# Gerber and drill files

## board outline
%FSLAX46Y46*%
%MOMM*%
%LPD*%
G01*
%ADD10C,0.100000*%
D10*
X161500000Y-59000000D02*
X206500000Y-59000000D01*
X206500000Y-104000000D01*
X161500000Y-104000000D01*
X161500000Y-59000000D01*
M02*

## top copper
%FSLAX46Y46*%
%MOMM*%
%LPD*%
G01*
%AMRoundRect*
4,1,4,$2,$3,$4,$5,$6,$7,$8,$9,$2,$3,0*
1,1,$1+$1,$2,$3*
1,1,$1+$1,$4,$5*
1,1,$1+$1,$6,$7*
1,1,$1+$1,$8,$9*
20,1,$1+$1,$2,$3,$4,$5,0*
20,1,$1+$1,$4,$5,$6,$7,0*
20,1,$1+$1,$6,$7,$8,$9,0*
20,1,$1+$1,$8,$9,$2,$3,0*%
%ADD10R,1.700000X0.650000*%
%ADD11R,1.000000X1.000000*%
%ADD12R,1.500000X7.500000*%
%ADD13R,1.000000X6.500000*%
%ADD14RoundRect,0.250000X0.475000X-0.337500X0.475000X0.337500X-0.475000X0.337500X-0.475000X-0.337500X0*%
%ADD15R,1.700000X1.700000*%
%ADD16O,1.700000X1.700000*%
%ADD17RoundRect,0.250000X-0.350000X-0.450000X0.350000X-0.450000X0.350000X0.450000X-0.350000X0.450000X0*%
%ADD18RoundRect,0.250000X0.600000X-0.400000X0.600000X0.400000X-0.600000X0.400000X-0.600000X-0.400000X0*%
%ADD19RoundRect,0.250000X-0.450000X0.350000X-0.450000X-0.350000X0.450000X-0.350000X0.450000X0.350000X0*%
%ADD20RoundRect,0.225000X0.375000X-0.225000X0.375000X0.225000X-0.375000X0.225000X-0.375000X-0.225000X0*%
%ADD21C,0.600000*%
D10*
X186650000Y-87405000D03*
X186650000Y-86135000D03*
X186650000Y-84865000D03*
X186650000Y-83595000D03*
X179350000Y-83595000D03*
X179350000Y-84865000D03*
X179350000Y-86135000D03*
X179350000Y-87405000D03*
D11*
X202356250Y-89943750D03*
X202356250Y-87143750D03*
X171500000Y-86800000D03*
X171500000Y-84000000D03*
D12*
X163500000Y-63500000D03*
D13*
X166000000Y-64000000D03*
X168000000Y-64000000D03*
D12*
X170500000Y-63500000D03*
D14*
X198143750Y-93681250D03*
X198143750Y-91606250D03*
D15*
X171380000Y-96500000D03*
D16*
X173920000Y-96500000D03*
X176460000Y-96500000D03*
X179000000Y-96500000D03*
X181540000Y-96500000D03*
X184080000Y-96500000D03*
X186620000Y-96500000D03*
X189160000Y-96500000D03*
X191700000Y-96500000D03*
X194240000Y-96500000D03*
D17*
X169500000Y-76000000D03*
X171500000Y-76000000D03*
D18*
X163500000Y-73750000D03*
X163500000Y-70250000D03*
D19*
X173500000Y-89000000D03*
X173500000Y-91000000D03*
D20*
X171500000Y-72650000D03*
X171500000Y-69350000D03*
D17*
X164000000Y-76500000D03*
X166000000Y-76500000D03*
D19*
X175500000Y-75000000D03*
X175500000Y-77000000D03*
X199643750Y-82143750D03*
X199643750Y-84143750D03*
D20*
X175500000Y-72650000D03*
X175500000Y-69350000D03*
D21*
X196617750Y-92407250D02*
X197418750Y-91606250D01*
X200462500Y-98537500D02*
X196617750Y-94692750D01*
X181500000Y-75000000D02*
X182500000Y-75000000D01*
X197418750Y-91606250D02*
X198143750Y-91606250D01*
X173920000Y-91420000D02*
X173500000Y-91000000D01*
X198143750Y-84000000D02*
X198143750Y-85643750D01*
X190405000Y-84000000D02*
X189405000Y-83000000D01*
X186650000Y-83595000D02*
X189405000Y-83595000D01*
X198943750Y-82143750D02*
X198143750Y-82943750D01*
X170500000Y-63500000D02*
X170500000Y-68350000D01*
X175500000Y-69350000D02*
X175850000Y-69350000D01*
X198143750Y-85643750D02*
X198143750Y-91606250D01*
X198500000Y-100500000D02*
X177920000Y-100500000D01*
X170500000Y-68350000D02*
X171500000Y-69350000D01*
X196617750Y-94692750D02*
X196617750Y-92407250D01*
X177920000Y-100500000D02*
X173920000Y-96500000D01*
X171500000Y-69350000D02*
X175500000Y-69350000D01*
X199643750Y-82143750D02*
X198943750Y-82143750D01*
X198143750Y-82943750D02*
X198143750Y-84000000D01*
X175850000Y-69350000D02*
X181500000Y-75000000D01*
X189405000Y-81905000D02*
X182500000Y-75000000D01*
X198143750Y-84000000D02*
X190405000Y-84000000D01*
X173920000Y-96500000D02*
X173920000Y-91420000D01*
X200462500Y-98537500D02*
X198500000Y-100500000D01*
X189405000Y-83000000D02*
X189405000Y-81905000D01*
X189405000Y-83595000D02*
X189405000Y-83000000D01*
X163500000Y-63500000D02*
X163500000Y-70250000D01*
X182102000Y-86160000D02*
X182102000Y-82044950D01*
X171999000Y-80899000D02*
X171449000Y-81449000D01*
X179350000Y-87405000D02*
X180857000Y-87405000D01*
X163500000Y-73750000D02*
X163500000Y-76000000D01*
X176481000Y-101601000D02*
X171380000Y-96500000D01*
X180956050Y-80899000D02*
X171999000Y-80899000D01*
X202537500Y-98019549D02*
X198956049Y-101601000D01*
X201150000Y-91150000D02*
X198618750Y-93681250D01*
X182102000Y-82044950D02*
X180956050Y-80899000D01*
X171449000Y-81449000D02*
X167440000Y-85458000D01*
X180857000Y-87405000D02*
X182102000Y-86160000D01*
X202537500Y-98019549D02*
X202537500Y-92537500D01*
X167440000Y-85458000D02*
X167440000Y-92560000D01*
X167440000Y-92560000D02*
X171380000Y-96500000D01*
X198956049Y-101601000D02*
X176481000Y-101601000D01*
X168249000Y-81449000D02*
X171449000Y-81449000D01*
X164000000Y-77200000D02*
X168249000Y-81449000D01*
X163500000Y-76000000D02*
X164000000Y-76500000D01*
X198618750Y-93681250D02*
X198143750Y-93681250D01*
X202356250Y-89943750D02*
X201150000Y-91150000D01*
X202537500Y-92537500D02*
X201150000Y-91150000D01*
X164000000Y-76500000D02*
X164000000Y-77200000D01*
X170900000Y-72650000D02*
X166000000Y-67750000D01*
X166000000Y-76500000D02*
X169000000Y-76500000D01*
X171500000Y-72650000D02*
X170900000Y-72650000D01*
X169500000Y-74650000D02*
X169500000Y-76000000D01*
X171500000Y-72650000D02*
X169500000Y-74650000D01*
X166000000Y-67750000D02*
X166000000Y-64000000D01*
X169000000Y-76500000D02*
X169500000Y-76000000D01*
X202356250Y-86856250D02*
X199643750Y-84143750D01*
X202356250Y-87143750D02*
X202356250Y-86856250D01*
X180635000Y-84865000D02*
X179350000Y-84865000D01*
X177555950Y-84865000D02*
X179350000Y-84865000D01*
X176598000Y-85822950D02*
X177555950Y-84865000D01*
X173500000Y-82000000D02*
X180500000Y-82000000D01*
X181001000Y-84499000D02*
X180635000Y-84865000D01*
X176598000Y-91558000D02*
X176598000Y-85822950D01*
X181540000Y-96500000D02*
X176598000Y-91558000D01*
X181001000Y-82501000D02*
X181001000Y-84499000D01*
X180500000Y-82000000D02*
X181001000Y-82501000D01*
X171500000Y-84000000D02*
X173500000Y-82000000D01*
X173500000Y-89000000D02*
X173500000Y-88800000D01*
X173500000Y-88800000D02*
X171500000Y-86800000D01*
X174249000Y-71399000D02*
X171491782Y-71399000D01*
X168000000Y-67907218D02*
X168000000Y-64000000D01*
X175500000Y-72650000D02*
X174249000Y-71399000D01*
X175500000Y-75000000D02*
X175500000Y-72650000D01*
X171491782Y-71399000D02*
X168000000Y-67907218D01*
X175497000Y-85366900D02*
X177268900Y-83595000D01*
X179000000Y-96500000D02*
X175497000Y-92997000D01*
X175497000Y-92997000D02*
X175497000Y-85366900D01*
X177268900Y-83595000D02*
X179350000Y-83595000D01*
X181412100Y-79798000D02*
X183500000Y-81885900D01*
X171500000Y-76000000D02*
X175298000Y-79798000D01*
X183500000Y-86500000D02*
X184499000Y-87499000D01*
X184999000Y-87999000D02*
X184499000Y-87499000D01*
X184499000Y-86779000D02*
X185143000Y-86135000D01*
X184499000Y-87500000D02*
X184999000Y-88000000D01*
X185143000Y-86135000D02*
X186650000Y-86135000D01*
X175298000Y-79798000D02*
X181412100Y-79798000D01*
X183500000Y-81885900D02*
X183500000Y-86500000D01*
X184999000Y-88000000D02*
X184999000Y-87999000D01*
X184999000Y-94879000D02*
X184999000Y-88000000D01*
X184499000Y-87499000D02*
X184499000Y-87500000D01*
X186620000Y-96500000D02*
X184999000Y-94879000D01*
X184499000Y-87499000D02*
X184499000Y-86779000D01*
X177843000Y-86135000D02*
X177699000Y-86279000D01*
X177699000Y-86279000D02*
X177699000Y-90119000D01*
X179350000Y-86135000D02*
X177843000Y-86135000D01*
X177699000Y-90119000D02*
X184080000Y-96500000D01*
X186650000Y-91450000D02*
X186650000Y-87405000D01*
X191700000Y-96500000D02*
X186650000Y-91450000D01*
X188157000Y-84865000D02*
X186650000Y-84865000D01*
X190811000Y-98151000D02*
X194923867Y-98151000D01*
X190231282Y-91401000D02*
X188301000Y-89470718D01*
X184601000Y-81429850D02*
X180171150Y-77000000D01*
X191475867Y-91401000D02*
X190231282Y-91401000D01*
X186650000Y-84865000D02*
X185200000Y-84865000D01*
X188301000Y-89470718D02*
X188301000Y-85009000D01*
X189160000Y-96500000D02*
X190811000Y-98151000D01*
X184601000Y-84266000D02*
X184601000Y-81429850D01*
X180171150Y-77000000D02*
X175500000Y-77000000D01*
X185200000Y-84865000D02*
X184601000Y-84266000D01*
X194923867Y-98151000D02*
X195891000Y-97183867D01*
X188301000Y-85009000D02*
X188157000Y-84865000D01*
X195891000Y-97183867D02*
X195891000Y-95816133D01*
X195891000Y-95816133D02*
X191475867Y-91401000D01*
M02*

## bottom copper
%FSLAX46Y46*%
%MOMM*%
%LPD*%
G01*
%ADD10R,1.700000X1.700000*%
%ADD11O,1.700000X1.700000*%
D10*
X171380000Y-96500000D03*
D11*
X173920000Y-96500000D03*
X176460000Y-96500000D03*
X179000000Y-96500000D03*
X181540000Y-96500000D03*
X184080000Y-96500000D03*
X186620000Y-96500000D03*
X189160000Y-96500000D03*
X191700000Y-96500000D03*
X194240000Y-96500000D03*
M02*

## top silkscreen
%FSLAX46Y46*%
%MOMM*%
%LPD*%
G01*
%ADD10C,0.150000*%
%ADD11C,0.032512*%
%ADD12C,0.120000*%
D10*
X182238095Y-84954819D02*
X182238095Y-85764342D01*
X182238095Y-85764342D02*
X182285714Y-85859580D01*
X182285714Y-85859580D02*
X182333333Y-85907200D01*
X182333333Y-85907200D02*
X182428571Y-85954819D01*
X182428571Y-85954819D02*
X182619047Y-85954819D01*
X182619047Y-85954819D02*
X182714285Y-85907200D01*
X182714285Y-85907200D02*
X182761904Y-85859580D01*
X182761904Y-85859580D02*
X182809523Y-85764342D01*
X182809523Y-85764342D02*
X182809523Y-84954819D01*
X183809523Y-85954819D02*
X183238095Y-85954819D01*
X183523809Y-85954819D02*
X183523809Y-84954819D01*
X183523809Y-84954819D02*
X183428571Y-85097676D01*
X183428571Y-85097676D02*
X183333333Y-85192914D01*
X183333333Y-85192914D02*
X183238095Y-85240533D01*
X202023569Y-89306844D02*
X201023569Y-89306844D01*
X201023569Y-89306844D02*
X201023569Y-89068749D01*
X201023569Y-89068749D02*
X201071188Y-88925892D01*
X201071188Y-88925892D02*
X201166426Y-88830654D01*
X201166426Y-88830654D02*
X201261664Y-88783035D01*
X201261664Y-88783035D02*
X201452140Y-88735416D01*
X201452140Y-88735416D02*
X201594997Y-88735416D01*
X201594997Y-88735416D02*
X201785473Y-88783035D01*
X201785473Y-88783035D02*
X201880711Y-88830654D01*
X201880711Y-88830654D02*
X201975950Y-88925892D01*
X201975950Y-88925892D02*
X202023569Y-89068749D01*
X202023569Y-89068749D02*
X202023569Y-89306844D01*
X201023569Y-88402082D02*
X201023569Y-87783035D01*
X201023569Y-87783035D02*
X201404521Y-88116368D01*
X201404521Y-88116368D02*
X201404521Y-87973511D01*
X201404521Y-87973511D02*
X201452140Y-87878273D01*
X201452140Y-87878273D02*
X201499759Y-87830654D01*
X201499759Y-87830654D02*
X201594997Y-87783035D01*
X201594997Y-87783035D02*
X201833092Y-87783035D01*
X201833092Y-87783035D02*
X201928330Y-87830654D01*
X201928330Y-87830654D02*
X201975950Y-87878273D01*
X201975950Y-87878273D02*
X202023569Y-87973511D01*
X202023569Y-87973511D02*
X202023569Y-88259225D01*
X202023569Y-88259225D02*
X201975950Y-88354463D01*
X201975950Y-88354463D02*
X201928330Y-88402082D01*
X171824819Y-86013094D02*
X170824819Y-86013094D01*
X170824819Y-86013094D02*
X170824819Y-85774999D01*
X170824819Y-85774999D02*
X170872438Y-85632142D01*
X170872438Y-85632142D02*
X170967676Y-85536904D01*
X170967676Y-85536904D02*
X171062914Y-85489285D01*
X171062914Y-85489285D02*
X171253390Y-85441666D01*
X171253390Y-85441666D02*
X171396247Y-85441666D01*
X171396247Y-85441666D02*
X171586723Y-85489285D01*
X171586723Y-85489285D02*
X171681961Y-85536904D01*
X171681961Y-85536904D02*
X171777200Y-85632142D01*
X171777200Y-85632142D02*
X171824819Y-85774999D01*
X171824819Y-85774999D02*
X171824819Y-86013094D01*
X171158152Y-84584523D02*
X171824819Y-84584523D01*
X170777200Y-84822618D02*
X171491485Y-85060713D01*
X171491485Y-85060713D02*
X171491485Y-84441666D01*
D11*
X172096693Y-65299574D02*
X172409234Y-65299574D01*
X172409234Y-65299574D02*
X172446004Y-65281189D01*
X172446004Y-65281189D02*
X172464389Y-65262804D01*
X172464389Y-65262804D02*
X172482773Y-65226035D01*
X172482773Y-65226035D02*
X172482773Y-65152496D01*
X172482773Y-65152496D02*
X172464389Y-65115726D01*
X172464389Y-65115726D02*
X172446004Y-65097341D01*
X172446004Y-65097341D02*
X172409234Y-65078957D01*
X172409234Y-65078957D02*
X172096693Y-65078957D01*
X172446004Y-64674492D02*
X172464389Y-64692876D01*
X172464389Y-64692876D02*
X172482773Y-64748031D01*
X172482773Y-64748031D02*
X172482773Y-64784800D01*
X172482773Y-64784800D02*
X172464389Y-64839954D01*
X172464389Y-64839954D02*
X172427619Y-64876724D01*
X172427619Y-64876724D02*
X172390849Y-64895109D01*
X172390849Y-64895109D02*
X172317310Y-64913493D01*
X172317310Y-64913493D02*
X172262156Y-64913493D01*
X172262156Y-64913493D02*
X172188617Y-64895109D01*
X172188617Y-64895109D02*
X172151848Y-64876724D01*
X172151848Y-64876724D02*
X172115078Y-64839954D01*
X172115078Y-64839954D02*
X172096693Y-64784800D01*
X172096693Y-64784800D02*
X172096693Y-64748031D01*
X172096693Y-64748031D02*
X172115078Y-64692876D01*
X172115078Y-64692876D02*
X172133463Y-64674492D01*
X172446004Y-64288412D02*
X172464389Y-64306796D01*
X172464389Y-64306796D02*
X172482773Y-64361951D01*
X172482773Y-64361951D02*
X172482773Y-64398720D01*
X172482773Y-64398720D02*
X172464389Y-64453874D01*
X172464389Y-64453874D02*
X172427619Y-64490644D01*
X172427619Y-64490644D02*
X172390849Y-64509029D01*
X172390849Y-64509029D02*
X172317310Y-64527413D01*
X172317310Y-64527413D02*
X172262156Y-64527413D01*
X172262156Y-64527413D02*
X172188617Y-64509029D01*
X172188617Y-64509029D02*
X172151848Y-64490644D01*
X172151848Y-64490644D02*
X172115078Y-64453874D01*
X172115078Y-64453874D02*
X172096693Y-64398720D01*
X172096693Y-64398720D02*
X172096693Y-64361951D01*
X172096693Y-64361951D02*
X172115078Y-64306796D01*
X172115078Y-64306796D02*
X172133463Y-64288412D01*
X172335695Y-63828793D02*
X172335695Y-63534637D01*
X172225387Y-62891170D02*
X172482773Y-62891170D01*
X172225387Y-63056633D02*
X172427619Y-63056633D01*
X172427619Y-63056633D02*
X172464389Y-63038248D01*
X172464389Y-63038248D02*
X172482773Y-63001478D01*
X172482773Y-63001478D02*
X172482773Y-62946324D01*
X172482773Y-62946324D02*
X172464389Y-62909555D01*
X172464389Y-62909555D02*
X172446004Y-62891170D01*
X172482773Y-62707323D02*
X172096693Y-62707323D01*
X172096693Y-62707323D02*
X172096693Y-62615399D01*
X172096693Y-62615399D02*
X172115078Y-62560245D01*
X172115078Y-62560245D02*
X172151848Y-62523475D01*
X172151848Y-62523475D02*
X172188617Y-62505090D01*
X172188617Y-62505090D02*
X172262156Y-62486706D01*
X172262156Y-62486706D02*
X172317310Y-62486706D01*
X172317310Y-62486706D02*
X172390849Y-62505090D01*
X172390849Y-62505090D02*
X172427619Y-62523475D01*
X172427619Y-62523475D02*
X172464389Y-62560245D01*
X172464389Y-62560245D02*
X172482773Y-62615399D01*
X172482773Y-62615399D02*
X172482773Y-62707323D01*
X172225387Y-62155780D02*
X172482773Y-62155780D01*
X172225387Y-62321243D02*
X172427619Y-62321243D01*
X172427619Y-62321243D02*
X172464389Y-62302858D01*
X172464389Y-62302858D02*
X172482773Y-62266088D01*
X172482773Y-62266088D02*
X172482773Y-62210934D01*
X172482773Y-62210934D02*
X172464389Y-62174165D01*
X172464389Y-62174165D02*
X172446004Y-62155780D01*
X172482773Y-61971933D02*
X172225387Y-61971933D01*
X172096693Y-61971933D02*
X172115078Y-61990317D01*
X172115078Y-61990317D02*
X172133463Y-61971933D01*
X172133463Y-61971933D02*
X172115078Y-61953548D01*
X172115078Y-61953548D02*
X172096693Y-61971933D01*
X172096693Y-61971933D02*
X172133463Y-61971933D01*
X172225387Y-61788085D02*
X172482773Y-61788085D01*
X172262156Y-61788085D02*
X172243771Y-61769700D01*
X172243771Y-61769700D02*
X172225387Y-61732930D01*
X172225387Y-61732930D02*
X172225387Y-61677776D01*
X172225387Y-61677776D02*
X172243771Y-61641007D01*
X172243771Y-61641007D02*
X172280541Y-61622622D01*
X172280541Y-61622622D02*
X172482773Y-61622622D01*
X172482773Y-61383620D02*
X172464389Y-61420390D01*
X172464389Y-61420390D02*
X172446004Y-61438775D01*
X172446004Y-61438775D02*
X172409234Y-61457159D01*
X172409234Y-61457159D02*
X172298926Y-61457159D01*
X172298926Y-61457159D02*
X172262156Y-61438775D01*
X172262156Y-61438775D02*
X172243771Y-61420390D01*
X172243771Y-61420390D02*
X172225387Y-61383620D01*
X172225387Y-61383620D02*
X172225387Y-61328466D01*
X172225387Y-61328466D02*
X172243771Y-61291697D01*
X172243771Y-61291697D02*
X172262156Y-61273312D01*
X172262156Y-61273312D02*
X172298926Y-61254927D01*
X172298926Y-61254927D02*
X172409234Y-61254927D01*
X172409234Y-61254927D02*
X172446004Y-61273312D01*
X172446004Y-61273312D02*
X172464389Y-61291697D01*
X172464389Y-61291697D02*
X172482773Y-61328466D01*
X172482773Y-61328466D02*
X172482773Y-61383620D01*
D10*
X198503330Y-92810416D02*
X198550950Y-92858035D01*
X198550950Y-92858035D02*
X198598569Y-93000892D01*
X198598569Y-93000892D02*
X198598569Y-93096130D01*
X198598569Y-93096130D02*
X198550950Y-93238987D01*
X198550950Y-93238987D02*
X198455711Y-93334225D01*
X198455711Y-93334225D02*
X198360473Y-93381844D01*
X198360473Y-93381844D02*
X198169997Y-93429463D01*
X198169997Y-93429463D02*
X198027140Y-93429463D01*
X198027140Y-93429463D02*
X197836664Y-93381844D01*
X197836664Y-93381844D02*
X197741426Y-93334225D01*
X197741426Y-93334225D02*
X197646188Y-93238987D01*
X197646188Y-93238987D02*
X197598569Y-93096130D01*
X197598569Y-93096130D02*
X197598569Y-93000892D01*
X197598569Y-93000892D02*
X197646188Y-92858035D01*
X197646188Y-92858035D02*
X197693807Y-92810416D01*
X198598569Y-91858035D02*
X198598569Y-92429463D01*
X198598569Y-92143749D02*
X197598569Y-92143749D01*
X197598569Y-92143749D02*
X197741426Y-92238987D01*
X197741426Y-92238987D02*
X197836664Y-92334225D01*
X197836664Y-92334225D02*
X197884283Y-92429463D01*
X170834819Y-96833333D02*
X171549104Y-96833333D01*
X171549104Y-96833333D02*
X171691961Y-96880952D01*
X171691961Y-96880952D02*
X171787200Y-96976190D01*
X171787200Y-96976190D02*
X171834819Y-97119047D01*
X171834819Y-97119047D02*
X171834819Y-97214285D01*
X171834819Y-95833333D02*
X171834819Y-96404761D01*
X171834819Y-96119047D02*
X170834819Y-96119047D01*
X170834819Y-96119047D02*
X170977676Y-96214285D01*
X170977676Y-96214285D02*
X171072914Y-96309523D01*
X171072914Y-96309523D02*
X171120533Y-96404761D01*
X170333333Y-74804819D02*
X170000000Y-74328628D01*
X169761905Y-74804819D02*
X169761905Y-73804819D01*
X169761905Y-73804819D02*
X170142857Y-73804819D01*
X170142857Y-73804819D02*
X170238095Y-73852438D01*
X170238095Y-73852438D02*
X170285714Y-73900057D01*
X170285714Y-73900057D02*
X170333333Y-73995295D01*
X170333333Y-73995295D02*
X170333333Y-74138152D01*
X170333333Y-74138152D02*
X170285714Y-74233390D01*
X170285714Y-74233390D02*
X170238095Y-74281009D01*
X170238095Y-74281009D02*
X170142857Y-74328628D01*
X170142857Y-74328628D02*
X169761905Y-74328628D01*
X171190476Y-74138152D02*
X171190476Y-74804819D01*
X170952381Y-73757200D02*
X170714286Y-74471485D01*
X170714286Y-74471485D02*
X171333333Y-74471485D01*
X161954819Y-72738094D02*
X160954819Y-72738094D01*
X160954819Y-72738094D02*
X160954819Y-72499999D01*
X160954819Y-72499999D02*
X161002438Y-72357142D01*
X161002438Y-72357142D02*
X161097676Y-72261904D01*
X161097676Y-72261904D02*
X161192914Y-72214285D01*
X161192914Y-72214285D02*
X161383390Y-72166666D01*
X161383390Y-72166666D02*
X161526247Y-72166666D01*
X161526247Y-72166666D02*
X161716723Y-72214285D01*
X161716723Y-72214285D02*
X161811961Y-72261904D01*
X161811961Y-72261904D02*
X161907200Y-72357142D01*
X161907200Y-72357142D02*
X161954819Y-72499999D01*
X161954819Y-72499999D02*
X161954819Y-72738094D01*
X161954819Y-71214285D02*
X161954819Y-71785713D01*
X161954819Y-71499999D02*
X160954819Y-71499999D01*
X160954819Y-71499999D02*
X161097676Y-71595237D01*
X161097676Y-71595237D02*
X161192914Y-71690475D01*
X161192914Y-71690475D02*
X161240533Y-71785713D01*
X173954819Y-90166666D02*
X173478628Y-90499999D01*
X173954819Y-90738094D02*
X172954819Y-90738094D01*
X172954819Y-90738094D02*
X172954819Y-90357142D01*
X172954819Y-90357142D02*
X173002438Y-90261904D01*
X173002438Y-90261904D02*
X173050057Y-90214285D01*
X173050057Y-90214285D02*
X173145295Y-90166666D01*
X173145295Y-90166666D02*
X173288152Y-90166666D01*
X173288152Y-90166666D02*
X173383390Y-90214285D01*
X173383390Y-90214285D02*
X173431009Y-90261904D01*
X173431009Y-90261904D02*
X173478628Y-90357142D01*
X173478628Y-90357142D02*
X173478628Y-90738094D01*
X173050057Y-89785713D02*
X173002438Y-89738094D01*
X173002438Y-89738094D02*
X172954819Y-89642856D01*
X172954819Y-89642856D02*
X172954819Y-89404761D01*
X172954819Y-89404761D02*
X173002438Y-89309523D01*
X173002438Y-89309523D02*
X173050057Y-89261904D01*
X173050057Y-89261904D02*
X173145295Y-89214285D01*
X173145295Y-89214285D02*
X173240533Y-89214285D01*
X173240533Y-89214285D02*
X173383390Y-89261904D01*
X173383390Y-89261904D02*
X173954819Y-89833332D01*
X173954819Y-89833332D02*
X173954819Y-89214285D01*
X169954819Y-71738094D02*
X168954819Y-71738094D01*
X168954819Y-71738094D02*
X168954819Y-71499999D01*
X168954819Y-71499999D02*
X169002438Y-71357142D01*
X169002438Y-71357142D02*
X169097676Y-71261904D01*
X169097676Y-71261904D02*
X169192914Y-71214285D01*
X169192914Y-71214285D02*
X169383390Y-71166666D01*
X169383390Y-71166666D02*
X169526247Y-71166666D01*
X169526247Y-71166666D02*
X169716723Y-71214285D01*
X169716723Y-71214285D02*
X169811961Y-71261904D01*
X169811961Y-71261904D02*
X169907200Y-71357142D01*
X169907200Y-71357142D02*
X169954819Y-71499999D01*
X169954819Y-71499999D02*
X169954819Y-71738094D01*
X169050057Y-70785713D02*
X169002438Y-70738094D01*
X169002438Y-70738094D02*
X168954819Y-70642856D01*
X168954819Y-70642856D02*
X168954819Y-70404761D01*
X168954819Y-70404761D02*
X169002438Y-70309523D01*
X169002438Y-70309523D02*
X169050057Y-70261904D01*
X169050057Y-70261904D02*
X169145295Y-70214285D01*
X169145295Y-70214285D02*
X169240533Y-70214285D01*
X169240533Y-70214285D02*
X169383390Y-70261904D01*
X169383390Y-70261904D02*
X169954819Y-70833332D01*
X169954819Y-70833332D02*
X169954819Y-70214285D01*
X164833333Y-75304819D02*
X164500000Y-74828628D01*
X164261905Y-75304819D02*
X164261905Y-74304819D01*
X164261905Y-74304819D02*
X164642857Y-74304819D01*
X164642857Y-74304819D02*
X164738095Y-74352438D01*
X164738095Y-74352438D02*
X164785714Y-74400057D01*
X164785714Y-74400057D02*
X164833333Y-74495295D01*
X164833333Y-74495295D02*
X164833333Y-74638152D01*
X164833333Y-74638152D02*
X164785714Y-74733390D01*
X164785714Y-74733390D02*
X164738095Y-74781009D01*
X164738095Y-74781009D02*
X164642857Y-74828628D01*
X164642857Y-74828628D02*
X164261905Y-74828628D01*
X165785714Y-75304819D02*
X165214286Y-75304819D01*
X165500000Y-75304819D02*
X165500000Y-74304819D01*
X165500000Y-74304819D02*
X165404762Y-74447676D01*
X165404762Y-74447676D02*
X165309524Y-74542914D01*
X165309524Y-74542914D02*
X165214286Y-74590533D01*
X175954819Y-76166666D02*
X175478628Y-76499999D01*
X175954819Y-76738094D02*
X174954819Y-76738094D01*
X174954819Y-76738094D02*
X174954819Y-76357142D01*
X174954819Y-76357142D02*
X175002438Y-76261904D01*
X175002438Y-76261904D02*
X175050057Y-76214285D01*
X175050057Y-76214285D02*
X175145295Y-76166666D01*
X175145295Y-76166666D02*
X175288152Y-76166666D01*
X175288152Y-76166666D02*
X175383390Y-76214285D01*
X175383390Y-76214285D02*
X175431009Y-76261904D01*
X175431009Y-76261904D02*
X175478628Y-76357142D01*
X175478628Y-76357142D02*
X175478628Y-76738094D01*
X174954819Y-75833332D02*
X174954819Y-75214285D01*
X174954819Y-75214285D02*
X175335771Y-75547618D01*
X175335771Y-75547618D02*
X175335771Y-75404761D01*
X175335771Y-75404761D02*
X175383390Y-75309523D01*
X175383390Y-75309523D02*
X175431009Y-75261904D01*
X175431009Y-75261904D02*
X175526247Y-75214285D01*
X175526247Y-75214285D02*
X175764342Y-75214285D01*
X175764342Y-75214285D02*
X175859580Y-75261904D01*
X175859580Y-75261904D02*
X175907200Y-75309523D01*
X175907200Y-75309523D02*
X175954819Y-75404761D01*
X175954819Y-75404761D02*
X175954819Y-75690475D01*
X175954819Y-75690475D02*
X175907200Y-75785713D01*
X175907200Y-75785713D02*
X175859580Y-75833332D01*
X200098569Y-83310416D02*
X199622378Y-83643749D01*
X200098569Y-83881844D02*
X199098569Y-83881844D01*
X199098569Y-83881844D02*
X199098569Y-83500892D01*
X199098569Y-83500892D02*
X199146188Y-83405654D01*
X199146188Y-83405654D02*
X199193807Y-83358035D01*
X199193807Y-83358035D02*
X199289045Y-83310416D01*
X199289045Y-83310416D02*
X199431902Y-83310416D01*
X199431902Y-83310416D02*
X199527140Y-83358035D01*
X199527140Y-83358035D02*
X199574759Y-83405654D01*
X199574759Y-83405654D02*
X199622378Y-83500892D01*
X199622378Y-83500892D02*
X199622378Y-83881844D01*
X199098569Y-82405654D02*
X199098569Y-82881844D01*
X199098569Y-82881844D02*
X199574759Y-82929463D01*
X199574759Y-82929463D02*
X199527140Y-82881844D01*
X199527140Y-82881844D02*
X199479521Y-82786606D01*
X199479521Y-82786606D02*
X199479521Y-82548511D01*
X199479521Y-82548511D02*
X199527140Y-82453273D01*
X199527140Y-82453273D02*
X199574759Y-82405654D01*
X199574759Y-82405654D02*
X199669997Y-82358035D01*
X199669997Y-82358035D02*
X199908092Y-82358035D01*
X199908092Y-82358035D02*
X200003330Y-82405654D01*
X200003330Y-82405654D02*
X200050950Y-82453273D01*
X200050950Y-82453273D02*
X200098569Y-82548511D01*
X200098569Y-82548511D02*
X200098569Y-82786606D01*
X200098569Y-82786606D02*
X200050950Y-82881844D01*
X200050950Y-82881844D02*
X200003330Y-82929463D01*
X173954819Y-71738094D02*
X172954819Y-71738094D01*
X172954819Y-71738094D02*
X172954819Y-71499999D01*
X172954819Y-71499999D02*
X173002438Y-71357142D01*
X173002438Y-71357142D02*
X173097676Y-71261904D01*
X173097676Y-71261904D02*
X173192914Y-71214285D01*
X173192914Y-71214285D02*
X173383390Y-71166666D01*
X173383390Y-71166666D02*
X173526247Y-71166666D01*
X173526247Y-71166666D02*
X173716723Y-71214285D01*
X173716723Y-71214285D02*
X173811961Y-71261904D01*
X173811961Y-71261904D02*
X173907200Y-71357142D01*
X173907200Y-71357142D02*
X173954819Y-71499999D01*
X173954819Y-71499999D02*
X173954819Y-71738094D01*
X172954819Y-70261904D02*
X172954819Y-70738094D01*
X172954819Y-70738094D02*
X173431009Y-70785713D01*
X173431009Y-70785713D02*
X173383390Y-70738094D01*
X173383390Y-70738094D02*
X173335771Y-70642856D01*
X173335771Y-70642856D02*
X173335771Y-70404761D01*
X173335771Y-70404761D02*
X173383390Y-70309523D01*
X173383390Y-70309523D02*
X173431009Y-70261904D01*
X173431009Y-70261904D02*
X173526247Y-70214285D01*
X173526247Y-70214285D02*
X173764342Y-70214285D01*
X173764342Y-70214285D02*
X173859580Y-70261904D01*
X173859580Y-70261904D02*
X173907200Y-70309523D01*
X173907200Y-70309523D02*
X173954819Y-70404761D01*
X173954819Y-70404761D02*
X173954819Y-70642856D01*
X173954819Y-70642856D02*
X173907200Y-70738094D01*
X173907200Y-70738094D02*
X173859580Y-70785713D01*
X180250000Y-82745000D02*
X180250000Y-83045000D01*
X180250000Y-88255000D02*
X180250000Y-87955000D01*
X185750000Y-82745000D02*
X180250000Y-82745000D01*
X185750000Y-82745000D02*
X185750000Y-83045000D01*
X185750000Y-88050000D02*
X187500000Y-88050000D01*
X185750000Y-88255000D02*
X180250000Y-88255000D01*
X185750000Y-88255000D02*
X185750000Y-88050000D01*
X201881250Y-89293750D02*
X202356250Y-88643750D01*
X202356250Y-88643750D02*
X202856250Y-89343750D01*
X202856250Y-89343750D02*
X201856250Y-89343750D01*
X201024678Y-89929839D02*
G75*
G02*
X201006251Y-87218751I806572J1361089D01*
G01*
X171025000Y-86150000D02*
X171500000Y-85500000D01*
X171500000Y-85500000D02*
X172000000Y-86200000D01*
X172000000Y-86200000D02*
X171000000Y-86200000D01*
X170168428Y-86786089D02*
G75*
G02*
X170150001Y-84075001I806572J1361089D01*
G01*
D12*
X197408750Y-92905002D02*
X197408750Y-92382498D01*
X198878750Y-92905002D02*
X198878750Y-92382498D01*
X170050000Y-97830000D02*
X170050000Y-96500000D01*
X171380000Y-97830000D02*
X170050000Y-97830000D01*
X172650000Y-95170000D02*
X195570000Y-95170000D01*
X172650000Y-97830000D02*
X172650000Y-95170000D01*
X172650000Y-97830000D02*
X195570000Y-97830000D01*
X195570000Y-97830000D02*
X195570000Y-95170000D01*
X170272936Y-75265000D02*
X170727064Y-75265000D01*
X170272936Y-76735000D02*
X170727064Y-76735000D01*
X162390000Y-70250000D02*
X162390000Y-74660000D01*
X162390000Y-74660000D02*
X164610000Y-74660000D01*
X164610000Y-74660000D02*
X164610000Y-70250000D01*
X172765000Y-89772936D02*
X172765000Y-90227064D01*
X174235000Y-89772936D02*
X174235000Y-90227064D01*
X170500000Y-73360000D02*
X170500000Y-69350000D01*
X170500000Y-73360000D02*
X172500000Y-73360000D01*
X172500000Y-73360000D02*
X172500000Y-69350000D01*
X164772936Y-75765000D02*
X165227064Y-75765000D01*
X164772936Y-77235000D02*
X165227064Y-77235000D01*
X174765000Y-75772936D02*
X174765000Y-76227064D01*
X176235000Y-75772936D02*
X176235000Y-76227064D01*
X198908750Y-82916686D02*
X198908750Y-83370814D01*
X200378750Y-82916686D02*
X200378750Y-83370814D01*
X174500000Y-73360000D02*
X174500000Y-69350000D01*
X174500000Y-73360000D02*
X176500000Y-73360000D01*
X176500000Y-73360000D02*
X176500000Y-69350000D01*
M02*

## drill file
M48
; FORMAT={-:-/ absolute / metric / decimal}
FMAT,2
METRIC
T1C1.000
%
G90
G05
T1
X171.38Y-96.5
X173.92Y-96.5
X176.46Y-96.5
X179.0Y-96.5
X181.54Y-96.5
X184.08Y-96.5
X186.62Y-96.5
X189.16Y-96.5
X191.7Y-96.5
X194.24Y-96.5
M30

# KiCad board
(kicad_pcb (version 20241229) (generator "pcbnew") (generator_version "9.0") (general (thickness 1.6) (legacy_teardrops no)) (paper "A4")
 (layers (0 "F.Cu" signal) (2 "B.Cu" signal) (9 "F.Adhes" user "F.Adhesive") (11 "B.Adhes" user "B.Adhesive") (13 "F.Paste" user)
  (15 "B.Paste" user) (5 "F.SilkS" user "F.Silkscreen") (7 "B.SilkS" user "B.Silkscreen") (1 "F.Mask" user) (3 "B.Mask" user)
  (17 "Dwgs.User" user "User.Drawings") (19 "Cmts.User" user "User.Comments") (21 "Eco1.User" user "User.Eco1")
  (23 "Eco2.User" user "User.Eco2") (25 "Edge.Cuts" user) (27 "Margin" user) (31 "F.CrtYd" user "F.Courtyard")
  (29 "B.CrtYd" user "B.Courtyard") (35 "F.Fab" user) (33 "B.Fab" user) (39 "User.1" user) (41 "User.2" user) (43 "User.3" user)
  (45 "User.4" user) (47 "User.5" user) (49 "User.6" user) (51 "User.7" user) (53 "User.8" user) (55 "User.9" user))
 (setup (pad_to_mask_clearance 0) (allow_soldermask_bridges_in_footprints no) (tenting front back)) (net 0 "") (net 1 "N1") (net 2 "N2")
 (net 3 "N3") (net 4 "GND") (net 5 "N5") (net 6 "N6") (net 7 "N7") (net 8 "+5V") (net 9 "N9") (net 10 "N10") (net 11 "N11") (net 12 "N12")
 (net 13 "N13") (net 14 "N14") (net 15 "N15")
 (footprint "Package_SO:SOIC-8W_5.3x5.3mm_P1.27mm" (layer "F.Cu") (at 183 85.5 180)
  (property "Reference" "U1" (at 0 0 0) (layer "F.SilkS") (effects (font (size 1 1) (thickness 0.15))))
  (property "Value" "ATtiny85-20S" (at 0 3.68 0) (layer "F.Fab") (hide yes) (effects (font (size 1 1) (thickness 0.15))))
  (fp_line (start 2.75 2.755) (end 2.75 2.455) (stroke (width 0.15) (type solid)) (layer "F.SilkS"))
  (fp_line (start 2.75 -2.755) (end 2.75 -2.455) (stroke (width 0.15) (type solid)) (layer "F.SilkS"))
  (fp_line (start -2.75 2.755) (end 2.75 2.755) (stroke (width 0.15) (type solid)) (layer "F.SilkS"))
  (fp_line (start -2.75 2.755) (end -2.75 2.455) (stroke (width 0.15) (type solid)) (layer "F.SilkS"))
  (fp_line (start -2.75 -2.55) (end -4.5 -2.55) (stroke (width 0.15) (type solid)) (layer "F.SilkS"))
  (fp_line (start -2.75 -2.755) (end 2.75 -2.755) (stroke (width 0.15) (type solid)) (layer "F.SilkS"))
  (fp_line (start -2.75 -2.755) (end -2.75 -2.55) (stroke (width 0.15) (type solid)) (layer "F.SilkS"))
  (pad "1" smd rect (at -3.65 -1.905 180) (size 1.7 0.65) (layers "F.Cu" "F.Mask" "F.Paste") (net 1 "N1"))
  (pad "2" smd rect (at -3.65 -0.635 180) (size 1.7 0.65) (layers "F.Cu" "F.Mask" "F.Paste") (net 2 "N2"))
  (pad "3" smd rect (at -3.65 0.635 180) (size 1.7 0.65) (layers "F.Cu" "F.Mask" "F.Paste") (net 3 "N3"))
  (pad "4" smd rect (at -3.65 1.905 180) (size 1.7 0.65) (layers "F.Cu" "F.Mask" "F.Paste") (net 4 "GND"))
  (pad "5" smd rect (at 3.65 1.905 180) (size 1.7 0.65) (layers "F.Cu" "F.Mask" "F.Paste") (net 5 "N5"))
  (pad "6" smd rect (at 3.65 0.635 180) (size 1.7 0.65) (layers "F.Cu" "F.Mask" "F.Paste") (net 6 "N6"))
  (pad "7" smd rect (at 3.65 -0.635 180) (size 1.7 0.65) (layers "F.Cu" "F.Mask" "F.Paste") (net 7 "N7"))
  (pad "8" smd rect (at 3.65 -1.905 180) (size 1.7 0.65) (layers "F.Cu" "F.Mask" "F.Paste") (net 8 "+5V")))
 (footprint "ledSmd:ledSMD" (layer "F.Cu") (at 202.35625 88.14375 90)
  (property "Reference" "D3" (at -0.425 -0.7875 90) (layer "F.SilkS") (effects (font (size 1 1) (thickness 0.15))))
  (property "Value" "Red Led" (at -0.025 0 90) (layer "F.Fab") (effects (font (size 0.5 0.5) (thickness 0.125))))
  (fp_line (start -1.15 -0.475) (end -0.5 0) (stroke (width 0.15) (type solid)) (layer "F.SilkS"))
  (fp_line (start -0.5 0) (end -1.2 0.5) (stroke (width 0.15) (type solid)) (layer "F.SilkS"))
  (fp_line (start -1.2 0.5) (end -1.2 -0.5) (stroke (width 0.15) (type solid)) (layer "F.SilkS"))
  (fp_arc (start -1.786089 -1.331572) (mid -0.435753 -2.107089) (end 0.924999 -1.349999) (stroke (width 0.15) (type solid))
   (layer "F.SilkS"))
  (pad "1" smd rect (at -1.8 0 90) (size 1 1) (layers "F.Cu" "F.Mask" "F.Paste") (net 8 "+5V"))
  (pad "2" smd rect (at 1 0 90) (size 1 1) (layers "F.Cu" "F.Mask" "F.Paste") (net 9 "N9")))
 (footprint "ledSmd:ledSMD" (layer "F.Cu") (at 171.5 85 90)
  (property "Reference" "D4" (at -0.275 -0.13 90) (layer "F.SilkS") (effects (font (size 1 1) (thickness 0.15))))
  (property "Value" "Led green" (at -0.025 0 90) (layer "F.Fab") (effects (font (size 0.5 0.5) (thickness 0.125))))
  (fp_line (start -1.15 -0.475) (end -0.5 0) (stroke (width 0.15) (type solid)) (layer "F.SilkS"))
  (fp_line (start -0.5 0) (end -1.2 0.5) (stroke (width 0.15) (type solid)) (layer "F.SilkS"))
  (fp_line (start -1.2 0.5) (end -1.2 -0.5) (stroke (width 0.15) (type solid)) (layer "F.SilkS"))
  (fp_arc (start -1.786089 -1.331572) (mid -0.435753 -2.107089) (end 0.924999 -1.349999) (stroke (width 0.15) (type solid))
   (layer "F.SilkS"))
  (pad "1" smd rect (at -1.8 0 90) (size 1 1) (layers "F.Cu" "F.Mask" "F.Paste") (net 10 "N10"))
  (pad "2" smd rect (at 1 0 90) (size 1 1) (layers "F.Cu" "F.Mask" "F.Paste") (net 6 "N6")))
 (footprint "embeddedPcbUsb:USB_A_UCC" (layer "F.Cu") (at 167 63.7 -90)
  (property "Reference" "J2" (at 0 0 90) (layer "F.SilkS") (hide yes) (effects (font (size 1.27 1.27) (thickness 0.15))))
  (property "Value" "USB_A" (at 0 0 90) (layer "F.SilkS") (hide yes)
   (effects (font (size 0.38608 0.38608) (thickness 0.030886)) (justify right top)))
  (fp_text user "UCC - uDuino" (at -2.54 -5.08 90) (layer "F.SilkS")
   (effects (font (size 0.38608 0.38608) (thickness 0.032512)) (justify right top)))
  (pad "1" smd rect (at -0.2 3.5 270) (size 7.5 1.5) (layers "F.Cu" "F.Mask" "F.Paste") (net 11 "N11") (solder_mask_margin 0.1016))
  (pad "2" smd rect (at 0.3 1 270) (size 6.5 1) (layers "F.Cu" "F.Mask" "F.Paste") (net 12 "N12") (solder_mask_margin 0.1016))
  (pad "3" smd rect (at 0.3 -1 270) (size 6.5 1) (layers "F.Cu" "F.Mask" "F.Paste") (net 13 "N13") (solder_mask_margin 0.1016))
  (pad "4" smd rect (at -0.2 -3.5 270) (size 7.5 1.5) (layers "F.Cu" "F.Mask" "F.Paste") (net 4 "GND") (solder_mask_margin 0.1016)))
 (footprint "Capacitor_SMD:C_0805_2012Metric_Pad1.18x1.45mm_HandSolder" (layer "F.Cu") (at 198.14375 92.64375 90)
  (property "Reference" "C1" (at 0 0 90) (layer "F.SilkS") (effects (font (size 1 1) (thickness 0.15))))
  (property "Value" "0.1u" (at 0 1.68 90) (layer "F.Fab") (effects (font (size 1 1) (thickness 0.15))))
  (fp_line (start -0.261252 -0.735) (end 0.261252 -0.735) (stroke (width 0.12) (type solid)) (layer "F.SilkS"))
  (fp_line (start -0.261252 0.735) (end 0.261252 0.735) (stroke (width 0.12) (type solid)) (layer "F.SilkS"))
  (pad "1" smd roundrect (at -1.0375 0 90) (size 1.175 1.45) (layers "F.Cu" "F.Mask" "F.Paste") (roundrect_rratio 0.212766) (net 8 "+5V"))
  (pad "2" smd roundrect (at 1.0375 0 90) (size 1.175 1.45) (layers "F.Cu" "F.Mask" "F.Paste") (roundrect_rratio 0.212766) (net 4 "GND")))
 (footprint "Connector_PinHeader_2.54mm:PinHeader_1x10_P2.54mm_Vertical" (layer "F.Cu") (at 171.38 96.5 90)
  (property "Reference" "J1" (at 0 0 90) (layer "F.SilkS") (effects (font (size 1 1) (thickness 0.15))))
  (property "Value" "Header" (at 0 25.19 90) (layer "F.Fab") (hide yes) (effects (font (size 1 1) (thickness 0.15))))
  (fp_line (start -1.33 -1.33) (end 0 -1.33) (stroke (width 0.12) (type solid)) (layer "F.SilkS"))
  (fp_line (start -1.33 0) (end -1.33 -1.33) (stroke (width 0.12) (type solid)) (layer "F.SilkS"))
  (fp_line (start 1.33 1.27) (end 1.33 24.19) (stroke (width 0.12) (type solid)) (layer "F.SilkS"))
  (fp_line (start -1.33 1.27) (end 1.33 1.27) (stroke (width 0.12) (type solid)) (layer "F.SilkS"))
  (fp_line (start -1.33 1.27) (end -1.33 24.19) (stroke (width 0.12) (type solid)) (layer "F.SilkS"))
  (fp_line (start -1.33 24.19) (end 1.33 24.19) (stroke (width 0.12) (type solid)) (layer "F.SilkS"))
  (pad "1" thru_hole rect (at 0 0 90) (size 1.7 1.7) (drill 1) (layers "*.Cu" "*.Mask") (remove_unused_layers no) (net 8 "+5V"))
  (pad "2" thru_hole oval (at 0 2.54 90) (size 1.7 1.7) (drill 1) (layers "*.Cu" "*.Mask") (remove_unused_layers no) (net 4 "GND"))
  (pad "3" thru_hole oval (at 0 5.08 90) (size 1.7 1.7) (drill 1) (layers "*.Cu" "*.Mask") (remove_unused_layers no) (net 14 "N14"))
  (pad "4" thru_hole oval (at 0 7.62 90) (size 1.7 1.7) (drill 1) (layers "*.Cu" "*.Mask") (remove_unused_layers no) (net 5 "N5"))
  (pad "5" thru_hole oval (at 0 10.16 90) (size 1.7 1.7) (drill 1) (layers "*.Cu" "*.Mask") (remove_unused_layers no) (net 6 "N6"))
  (pad "6" thru_hole oval (at 0 12.7 90) (size 1.7 1.7) (drill 1) (layers "*.Cu" "*.Mask") (remove_unused_layers no) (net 7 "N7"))
  (pad "7" thru_hole oval (at 0 15.24 90) (size 1.7 1.7) (drill 1) (layers "*.Cu" "*.Mask") (remove_unused_layers no) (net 2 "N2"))
  (pad "8" thru_hole oval (at 0 17.78 90) (size 1.7 1.7) (drill 1) (layers "*.Cu" "*.Mask") (remove_unused_layers no) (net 3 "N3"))
  (pad "9" thru_hole oval (at 0 20.32 90) (size 1.7 1.7) (drill 1) (layers "*.Cu" "*.Mask") (remove_unused_layers no) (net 1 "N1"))
  (pad "10" thru_hole oval (at 0 22.86 90) (size 1.7 1.7) (drill 1) (layers "*.Cu" "*.Mask") (remove_unused_layers no) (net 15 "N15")))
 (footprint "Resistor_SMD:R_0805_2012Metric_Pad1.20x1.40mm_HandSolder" (layer "F.Cu") (at 170.5 76)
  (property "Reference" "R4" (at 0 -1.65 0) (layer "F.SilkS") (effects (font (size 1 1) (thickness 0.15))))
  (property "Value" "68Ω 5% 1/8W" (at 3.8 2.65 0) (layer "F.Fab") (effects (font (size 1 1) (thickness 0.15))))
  (fp_line (start -0.227064 -0.735) (end 0.227064 -0.735) (stroke (width 0.12) (type solid)) (layer "F.SilkS"))
  (fp_line (start -0.227064 0.735) (end 0.227064 0.735) (stroke (width 0.12) (type solid)) (layer "F.SilkS"))
  (pad "1" smd roundrect (at -1 0) (size 1.2 1.4) (layers "F.Cu" "F.Mask" "F.Paste") (roundrect_rratio 0.208333) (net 12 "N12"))
  (pad "2" smd roundrect (at 1 0) (size 1.2 1.4) (layers "F.Cu" "F.Mask" "F.Paste") (roundrect_rratio 0.208333) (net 2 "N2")))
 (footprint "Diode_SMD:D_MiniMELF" (layer "F.Cu") (at 163.5 72 90)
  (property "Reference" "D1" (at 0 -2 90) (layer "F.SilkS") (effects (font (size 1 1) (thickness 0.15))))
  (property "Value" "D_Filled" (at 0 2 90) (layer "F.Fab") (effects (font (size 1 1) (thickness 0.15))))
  (fp_line (start 1.75 -1.11) (end -2.66 -1.11) (stroke (width 0.12) (type solid)) (layer "F.SilkS"))
  (fp_line (start -2.66 -1.11) (end -2.66 1.11) (stroke (width 0.12) (type solid)) (layer "F.SilkS"))
  (fp_line (start -2.66 1.11) (end 1.75 1.11) (stroke (width 0.12) (type solid)) (layer "F.SilkS"))
  (pad "1" smd roundrect (at -1.75 0 90) (size 1.3 1.7) (layers "F.Cu" "F.Mask" "F.Paste") (roundrect_rratio 0.1923076923) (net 8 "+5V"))
  (pad "2" smd roundrect (at 1.75 0 90) (size 1.3 1.7) (layers "F.Cu" "F.Mask" "F.Paste") (roundrect_rratio 0.1923076923) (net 11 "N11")))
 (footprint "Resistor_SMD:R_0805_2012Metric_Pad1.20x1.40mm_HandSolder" (layer "F.Cu") (at 173.5 90 -90)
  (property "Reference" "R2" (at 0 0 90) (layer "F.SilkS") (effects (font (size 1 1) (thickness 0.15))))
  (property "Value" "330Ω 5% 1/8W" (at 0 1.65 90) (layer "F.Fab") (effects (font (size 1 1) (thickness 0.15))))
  (fp_line (start -0.227064 0.735) (end 0.227064 0.735) (stroke (width 0.12) (type solid)) (layer "F.SilkS"))
  (fp_line (start -0.227064 -0.735) (end 0.227064 -0.735) (stroke (width 0.12) (type solid)) (layer "F.SilkS"))
  (pad "1" smd roundrect (at -1 0 270) (size 1.2 1.4) (layers "F.Cu" "F.Mask" "F.Paste") (roundrect_rratio 0.208333) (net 10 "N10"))
  (pad "2" smd roundrect (at 1 0 270) (size 1.2 1.4) (layers "F.Cu" "F.Mask" "F.Paste") (roundrect_rratio 0.208333) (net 4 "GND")))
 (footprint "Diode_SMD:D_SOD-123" (layer "F.Cu") (at 171.5 71 90)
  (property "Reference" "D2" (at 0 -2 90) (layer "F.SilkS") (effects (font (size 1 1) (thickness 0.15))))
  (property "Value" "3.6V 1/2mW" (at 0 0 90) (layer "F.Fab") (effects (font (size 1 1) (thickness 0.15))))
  (fp_line (start -2.36 -1) (end 1.65 -1) (stroke (width 0.12) (type solid)) (layer "F.SilkS"))
  (fp_line (start -2.36 -1) (end -2.36 1) (stroke (width 0.12) (type solid)) (layer "F.SilkS"))
  (fp_line (start -2.36 1) (end 1.65 1) (stroke (width 0.12) (type solid)) (layer "F.SilkS"))
  (pad "1" smd roundrect (at -1.65 0 90) (size 0.9 1.2) (layers "F.Cu" "F.Mask" "F.Paste") (roundrect_rratio 0.25) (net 12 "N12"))
  (pad "2" smd roundrect (at 1.65 0 90) (size 0.9 1.2) (layers "F.Cu" "F.Mask" "F.Paste") (roundrect_rratio 0.25) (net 4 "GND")))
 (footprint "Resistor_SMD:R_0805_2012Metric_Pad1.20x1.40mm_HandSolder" (layer "F.Cu") (at 165 76.5)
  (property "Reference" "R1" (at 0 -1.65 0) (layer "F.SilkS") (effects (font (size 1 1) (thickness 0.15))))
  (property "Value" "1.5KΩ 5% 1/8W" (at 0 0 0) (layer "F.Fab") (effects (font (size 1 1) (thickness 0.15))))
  (fp_line (start -0.227064 -0.735) (end 0.227064 -0.735) (stroke (width 0.12) (type solid)) (layer "F.SilkS"))
  (fp_line (start -0.227064 0.735) (end 0.227064 0.735) (stroke (width 0.12) (type solid)) (layer "F.SilkS"))
  (pad "1" smd roundrect (at -1 0) (size 1.2 1.4) (layers "F.Cu" "F.Mask" "F.Paste") (roundrect_rratio 0.208333) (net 8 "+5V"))
  (pad "2" smd roundrect (at 1 0) (size 1.2 1.4) (layers "F.Cu" "F.Mask" "F.Paste") (roundrect_rratio 0.208333) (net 12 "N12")))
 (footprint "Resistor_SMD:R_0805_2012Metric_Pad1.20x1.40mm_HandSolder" (layer "F.Cu") (at 175.5 76 -90)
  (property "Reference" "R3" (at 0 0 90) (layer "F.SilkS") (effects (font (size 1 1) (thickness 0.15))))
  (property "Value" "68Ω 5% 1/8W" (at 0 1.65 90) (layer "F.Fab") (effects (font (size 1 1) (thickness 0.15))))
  (fp_line (start -0.227064 0.735) (end 0.227064 0.735) (stroke (width 0.12) (type solid)) (layer "F.SilkS"))
  (fp_line (start -0.227064 -0.735) (end 0.227064 -0.735) (stroke (width 0.12) (type solid)) (layer "F.SilkS"))
  (pad "1" smd roundrect (at -1 0 270) (size 1.2 1.4) (layers "F.Cu" "F.Mask" "F.Paste") (roundrect_rratio 0.208333) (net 13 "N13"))
  (pad "2" smd roundrect (at 1 0 270) (size 1.2 1.4) (layers "F.Cu" "F.Mask" "F.Paste") (roundrect_rratio 0.208333) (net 3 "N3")))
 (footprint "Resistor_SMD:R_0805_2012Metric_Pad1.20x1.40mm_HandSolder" (layer "F.Cu") (at 199.64375 83.14375 -90)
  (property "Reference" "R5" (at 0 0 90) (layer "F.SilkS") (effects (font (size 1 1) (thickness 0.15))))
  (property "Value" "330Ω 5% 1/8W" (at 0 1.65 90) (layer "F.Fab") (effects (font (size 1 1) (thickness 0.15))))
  (fp_line (start -0.227064 0.735) (end 0.227064 0.735) (stroke (width 0.12) (type solid)) (layer "F.SilkS"))
  (fp_line (start -0.227064 -0.735) (end 0.227064 -0.735) (stroke (width 0.12) (type solid)) (layer "F.SilkS"))
  (pad "1" smd roundrect (at -1 0 270) (size 1.2 1.4) (layers "F.Cu" "F.Mask" "F.Paste") (roundrect_rratio 0.208333) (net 4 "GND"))
  (pad "2" smd roundrect (at 1 0 270) (size 1.2 1.4) (layers "F.Cu" "F.Mask" "F.Paste") (roundrect_rratio 0.208333) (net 9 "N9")))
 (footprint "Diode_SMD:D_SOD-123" (layer "F.Cu") (at 175.5 71 90)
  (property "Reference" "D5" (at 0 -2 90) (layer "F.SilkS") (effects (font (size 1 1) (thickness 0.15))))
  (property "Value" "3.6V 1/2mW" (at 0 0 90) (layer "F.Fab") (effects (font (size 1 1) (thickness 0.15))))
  (fp_line (start -2.36 -1) (end 1.65 -1) (stroke (width 0.12) (type solid)) (layer "F.SilkS"))
  (fp_line (start -2.36 -1) (end -2.36 1) (stroke (width 0.12) (type solid)) (layer "F.SilkS"))
  (fp_line (start -2.36 1) (end 1.65 1) (stroke (width 0.12) (type solid)) (layer "F.SilkS"))
  (pad "1" smd roundrect (at -1.65 0 90) (size 0.9 1.2) (layers "F.Cu" "F.Mask" "F.Paste") (roundrect_rratio 0.25) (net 13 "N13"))
  (pad "2" smd roundrect (at 1.65 0 90) (size 0.9 1.2) (layers "F.Cu" "F.Mask" "F.Paste") (roundrect_rratio 0.25) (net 4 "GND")))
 (gr_rect (start 161.5 59) (end 206.5 104) (stroke (width 0.1) (type default)) (fill no) (layer "Edge.Cuts"))
 (segment (start 196.61775 92.40725) (end 197.41875 91.60625) (width 0.6) (layer "F.Cu") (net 4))
 (segment (start 200.4625 98.5375) (end 196.61775 94.69275) (width 0.6) (layer "F.Cu") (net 4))
 (segment (start 181.5 75) (end 182.5 75) (width 0.6) (layer "F.Cu") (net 4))
 (segment (start 197.41875 91.60625) (end 198.14375 91.60625) (width 0.6) (layer "F.Cu") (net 4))
 (segment (start 173.92 91.42) (end 173.5 91) (width 0.6) (layer "F.Cu") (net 4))
 (segment (start 198.14375 84) (end 198.14375 85.64375) (width 0.6) (layer "F.Cu") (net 4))
 (segment (start 190.405 84) (end 189.405 83) (width 0.6) (layer "F.Cu") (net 4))
 (segment (start 186.65 83.595) (end 189.405 83.595) (width 0.6) (layer "F.Cu") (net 4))
 (segment (start 198.94375 82.14375) (end 198.14375 82.94375) (width 0.6) (layer "F.Cu") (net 4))
 (segment (start 170.5 63.5) (end 170.5 68.35) (width 0.6) (layer "F.Cu") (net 4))
 (segment (start 175.5 69.35) (end 175.85 69.35) (width 0.6) (layer "F.Cu") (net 4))
 (segment (start 198.14375 85.64375) (end 198.14375 91.60625) (width 0.6) (layer "F.Cu") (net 4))
 (segment (start 198.5 100.5) (end 177.92 100.5) (width 0.6) (layer "F.Cu") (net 4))
 (segment (start 170.5 68.35) (end 171.5 69.35) (width 0.6) (layer "F.Cu") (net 4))
 (segment (start 196.61775 94.69275) (end 196.61775 92.40725) (width 0.6) (layer "F.Cu") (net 4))
 (segment (start 177.92 100.5) (end 173.92 96.5) (width 0.6) (layer "F.Cu") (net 4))
 (segment (start 171.5 69.35) (end 175.5 69.35) (width 0.6) (layer "F.Cu") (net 4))
 (segment (start 199.64375 82.14375) (end 198.94375 82.14375) (width 0.6) (layer "F.Cu") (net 4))
 (segment (start 198.14375 82.94375) (end 198.14375 84) (width 0.6) (layer "F.Cu") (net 4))
 (segment (start 175.85 69.35) (end 181.5 75) (width 0.6) (layer "F.Cu") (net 4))
 (segment (start 189.405 81.905) (end 182.5 75) (width 0.6) (layer "F.Cu") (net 4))
 (segment (start 198.14375 84) (end 190.405 84) (width 0.6) (layer "F.Cu") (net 4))
 (segment (start 173.92 96.5) (end 173.92 91.42) (width 0.6) (layer "F.Cu") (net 4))
 (segment (start 200.4625 98.5375) (end 198.5 100.5) (width 0.6) (layer "F.Cu") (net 4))
 (segment (start 189.405 83) (end 189.405 81.905) (width 0.6) (layer "F.Cu") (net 4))
 (segment (start 189.405 83.595) (end 189.405 83) (width 0.6) (layer "F.Cu") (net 4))
 (segment (start 163.5 63.5) (end 163.5 70.25) (width 0.6) (layer "F.Cu") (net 11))
 (segment (start 182.102 86.16) (end 182.102 82.04495) (width 0.6) (layer "F.Cu") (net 8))
 (segment (start 171.999 80.899) (end 171.449 81.449) (width 0.6) (layer "F.Cu") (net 8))
 (segment (start 179.35 87.405) (end 180.857 87.405) (width 0.6) (layer "F.Cu") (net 8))
 (segment (start 163.5 73.75) (end 163.5 76) (width 0.6) (layer "F.Cu") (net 8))
 (segment (start 176.481 101.601) (end 171.38 96.5) (width 0.6) (layer "F.Cu") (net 8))
 (segment (start 180.95605 80.899) (end 171.999 80.899) (width 0.6) (layer "F.Cu") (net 8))
 (segment (start 202.5375 98.019549) (end 198.956049 101.601) (width 0.6) (layer "F.Cu") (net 8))
 (segment (start 201.15 91.15) (end 198.61875 93.68125) (width 0.6) (layer "F.Cu") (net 8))
 (segment (start 182.102 82.04495) (end 180.95605 80.899) (width 0.6) (layer "F.Cu") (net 8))
 (segment (start 171.449 81.449) (end 167.44 85.458) (width 0.6) (layer "F.Cu") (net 8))
 (segment (start 180.857 87.405) (end 182.102 86.16) (width 0.6) (layer "F.Cu") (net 8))
 (segment (start 202.5375 98.019549) (end 202.5375 92.5375) (width 0.6) (layer "F.Cu") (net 8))
 (segment (start 167.44 85.458) (end 167.44 92.56) (width 0.6) (layer "F.Cu") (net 8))
 (segment (start 167.44 92.56) (end 171.38 96.5) (width 0.6) (layer "F.Cu") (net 8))
 (segment (start 198.956049 101.601) (end 176.481 101.601) (width 0.6) (layer "F.Cu") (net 8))
 (segment (start 168.249 81.449) (end 171.449 81.449) (width 0.6) (layer "F.Cu") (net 8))
 (segment (start 164 77.2) (end 168.249 81.449) (width 0.6) (layer "F.Cu") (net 8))
 (segment (start 163.5 76) (end 164 76.5) (width 0.6) (layer "F.Cu") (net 8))
 (segment (start 198.61875 93.68125) (end 198.14375 93.68125) (width 0.6) (layer "F.Cu") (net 8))
 (segment (start 202.35625 89.94375) (end 201.15 91.15) (width 0.6) (layer "F.Cu") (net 8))
 (segment (start 202.5375 92.5375) (end 201.15 91.15) (width 0.6) (layer "F.Cu") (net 8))
 (segment (start 164 76.5) (end 164 77.2) (width 0.6) (layer "F.Cu") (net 8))
 (segment (start 170.9 72.65) (end 166 67.75) (width 0.6) (layer "F.Cu") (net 12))
 (segment (start 166 76.5) (end 169 76.5) (width 0.6) (layer "F.Cu") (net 12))
 (segment (start 171.5 72.65) (end 170.9 72.65) (width 0.6) (layer "F.Cu") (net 12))
 (segment (start 169.5 74.65) (end 169.5 76) (width 0.6) (layer "F.Cu") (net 12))
 (segment (start 171.5 72.65) (end 169.5 74.65) (width 0.6) (layer "F.Cu") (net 12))
 (segment (start 166 67.75) (end 166 64) (width 0.6) (layer "F.Cu") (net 12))
 (segment (start 169 76.5) (end 169.5 76) (width 0.6) (layer "F.Cu") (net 12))
 (segment (start 202.35625 86.85625) (end 199.64375 84.14375) (width 0.6) (layer "F.Cu") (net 9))
 (segment (start 202.35625 87.14375) (end 202.35625 86.85625) (width 0.6) (layer "F.Cu") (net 9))
 (segment (start 180.635 84.865) (end 179.35 84.865) (width 0.6) (layer "F.Cu") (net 6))
 (segment (start 177.55595 84.865) (end 179.35 84.865) (width 0.6) (layer "F.Cu") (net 6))
 (segment (start 176.598 85.82295) (end 177.55595 84.865) (width 0.6) (layer "F.Cu") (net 6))
 (segment (start 173.5 82) (end 180.5 82) (width 0.6) (layer "F.Cu") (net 6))
 (segment (start 181.001 84.499) (end 180.635 84.865) (width 0.6) (layer "F.Cu") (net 6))
 (segment (start 176.598 91.558) (end 176.598 85.82295) (width 0.6) (layer "F.Cu") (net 6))
 (segment (start 181.54 96.5) (end 176.598 91.558) (width 0.6) (layer "F.Cu") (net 6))
 (segment (start 181.001 82.501) (end 181.001 84.499) (width 0.6) (layer "F.Cu") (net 6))
 (segment (start 180.5 82) (end 181.001 82.501) (width 0.6) (layer "F.Cu") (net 6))
 (segment (start 171.5 84) (end 173.5 82) (width 0.6) (layer "F.Cu") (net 6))
 (segment (start 173.5 89) (end 173.5 88.8) (width 0.6) (layer "F.Cu") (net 10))
 (segment (start 173.5 88.8) (end 171.5 86.8) (width 0.6) (layer "F.Cu") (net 10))
 (segment (start 174.249 71.399) (end 171.491782 71.399) (width 0.6) (layer "F.Cu") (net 13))
 (segment (start 168 67.907218) (end 168 64) (width 0.6) (layer "F.Cu") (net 13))
 (segment (start 175.5 72.65) (end 174.249 71.399) (width 0.6) (layer "F.Cu") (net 13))
 (segment (start 175.5 75) (end 175.5 72.65) (width 0.6) (layer "F.Cu") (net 13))
 (segment (start 171.491782 71.399) (end 168 67.907218) (width 0.6) (layer "F.Cu") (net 13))
 (segment (start 175.497 85.3669) (end 177.2689 83.595) (width 0.6) (layer "F.Cu") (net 5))
 (segment (start 179 96.5) (end 175.497 92.997) (width 0.6) (layer "F.Cu") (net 5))
 (segment (start 175.497 92.997) (end 175.497 85.3669) (width 0.6) (layer "F.Cu") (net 5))
 (segment (start 177.2689 83.595) (end 179.35 83.595) (width 0.6) (layer "F.Cu") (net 5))
 (segment (start 181.4121 79.798) (end 183.5 81.8859) (width 0.6) (layer "F.Cu") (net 2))
 (segment (start 171.5 76) (end 175.298 79.798) (width 0.6) (layer "F.Cu") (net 2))
 (segment (start 183.5 86.5) (end 184.499 87.499) (width 0.6) (layer "F.Cu") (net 2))
 (segment (start 184.999 87.999) (end 184.499 87.499) (width 0.6) (layer "F.Cu") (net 2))
 (segment (start 184.499 86.779) (end 185.143 86.135) (width 0.6) (layer "F.Cu") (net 2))
 (segment (start 184.499 87.5) (end 184.999 88) (width 0.6) (layer "F.Cu") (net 2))
 (segment (start 185.143 86.135) (end 186.65 86.135) (width 0.6) (layer "F.Cu") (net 2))
 (segment (start 175.298 79.798) (end 181.4121 79.798) (width 0.6) (layer "F.Cu") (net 2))
 (segment (start 183.5 81.8859) (end 183.5 86.5) (width 0.6) (layer "F.Cu") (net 2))
 (segment (start 184.999 88) (end 184.999 87.999) (width 0.6) (layer "F.Cu") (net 2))
 (segment (start 184.999 94.879) (end 184.999 88) (width 0.6) (layer "F.Cu") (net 2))
 (segment (start 184.499 87.499) (end 184.499 87.5) (width 0.6) (layer "F.Cu") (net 2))
 (segment (start 186.62 96.5) (end 184.999 94.879) (width 0.6) (layer "F.Cu") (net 2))
 (segment (start 184.499 87.499) (end 184.499 86.779) (width 0.6) (layer "F.Cu") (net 2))
 (segment (start 177.843 86.135) (end 177.699 86.279) (width 0.6) (layer "F.Cu") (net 7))
 (segment (start 177.699 86.279) (end 177.699 90.119) (width 0.6) (layer "F.Cu") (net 7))
 (segment (start 179.35 86.135) (end 177.843 86.135) (width 0.6) (layer "F.Cu") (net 7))
 (segment (start 177.699 90.119) (end 184.08 96.5) (width 0.6) (layer "F.Cu") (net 7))
 (segment (start 186.65 91.45) (end 186.65 87.405) (width 0.6) (layer "F.Cu") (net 1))
 (segment (start 191.7 96.5) (end 186.65 91.45) (width 0.6) (layer "F.Cu") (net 1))
 (segment (start 188.157 84.865) (end 186.65 84.865) (width 0.6) (layer "F.Cu") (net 3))
 (segment (start 190.811 98.151) (end 194.923867 98.151) (width 0.6) (layer "F.Cu") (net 3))
 (segment (start 190.231282 91.401) (end 188.301 89.470718) (width 0.6) (layer "F.Cu") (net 3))
 (segment (start 184.601 81.42985) (end 180.17115 77) (width 0.6) (layer "F.Cu") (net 3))
 (segment (start 191.475867 91.401) (end 190.231282 91.401) (width 0.6) (layer "F.Cu") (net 3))
 (segment (start 186.65 84.865) (end 185.2 84.865) (width 0.6) (layer "F.Cu") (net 3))
 (segment (start 188.301 89.470718) (end 188.301 85.009) (width 0.6) (layer "F.Cu") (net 3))
 (segment (start 189.16 96.5) (end 190.811 98.151) (width 0.6) (layer "F.Cu") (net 3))
 (segment (start 184.601 84.266) (end 184.601 81.42985) (width 0.6) (layer "F.Cu") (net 3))
 (segment (start 180.17115 77) (end 175.5 77) (width 0.6) (layer "F.Cu") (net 3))
 (segment (start 185.2 84.865) (end 184.601 84.266) (width 0.6) (layer "F.Cu") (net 3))
 (segment (start 194.923867 98.151) (end 195.891 97.183867) (width 0.6) (layer "F.Cu") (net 3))
 (segment (start 188.301 85.009) (end 188.157 84.865) (width 0.6) (layer "F.Cu") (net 3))
 (segment (start 195.891 97.183867) (end 195.891 95.816133) (width 0.6) (layer "F.Cu") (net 3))
 (segment (start 195.891 95.816133) (end 191.475867 91.401) (width 0.6) (layer "F.Cu") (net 3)))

